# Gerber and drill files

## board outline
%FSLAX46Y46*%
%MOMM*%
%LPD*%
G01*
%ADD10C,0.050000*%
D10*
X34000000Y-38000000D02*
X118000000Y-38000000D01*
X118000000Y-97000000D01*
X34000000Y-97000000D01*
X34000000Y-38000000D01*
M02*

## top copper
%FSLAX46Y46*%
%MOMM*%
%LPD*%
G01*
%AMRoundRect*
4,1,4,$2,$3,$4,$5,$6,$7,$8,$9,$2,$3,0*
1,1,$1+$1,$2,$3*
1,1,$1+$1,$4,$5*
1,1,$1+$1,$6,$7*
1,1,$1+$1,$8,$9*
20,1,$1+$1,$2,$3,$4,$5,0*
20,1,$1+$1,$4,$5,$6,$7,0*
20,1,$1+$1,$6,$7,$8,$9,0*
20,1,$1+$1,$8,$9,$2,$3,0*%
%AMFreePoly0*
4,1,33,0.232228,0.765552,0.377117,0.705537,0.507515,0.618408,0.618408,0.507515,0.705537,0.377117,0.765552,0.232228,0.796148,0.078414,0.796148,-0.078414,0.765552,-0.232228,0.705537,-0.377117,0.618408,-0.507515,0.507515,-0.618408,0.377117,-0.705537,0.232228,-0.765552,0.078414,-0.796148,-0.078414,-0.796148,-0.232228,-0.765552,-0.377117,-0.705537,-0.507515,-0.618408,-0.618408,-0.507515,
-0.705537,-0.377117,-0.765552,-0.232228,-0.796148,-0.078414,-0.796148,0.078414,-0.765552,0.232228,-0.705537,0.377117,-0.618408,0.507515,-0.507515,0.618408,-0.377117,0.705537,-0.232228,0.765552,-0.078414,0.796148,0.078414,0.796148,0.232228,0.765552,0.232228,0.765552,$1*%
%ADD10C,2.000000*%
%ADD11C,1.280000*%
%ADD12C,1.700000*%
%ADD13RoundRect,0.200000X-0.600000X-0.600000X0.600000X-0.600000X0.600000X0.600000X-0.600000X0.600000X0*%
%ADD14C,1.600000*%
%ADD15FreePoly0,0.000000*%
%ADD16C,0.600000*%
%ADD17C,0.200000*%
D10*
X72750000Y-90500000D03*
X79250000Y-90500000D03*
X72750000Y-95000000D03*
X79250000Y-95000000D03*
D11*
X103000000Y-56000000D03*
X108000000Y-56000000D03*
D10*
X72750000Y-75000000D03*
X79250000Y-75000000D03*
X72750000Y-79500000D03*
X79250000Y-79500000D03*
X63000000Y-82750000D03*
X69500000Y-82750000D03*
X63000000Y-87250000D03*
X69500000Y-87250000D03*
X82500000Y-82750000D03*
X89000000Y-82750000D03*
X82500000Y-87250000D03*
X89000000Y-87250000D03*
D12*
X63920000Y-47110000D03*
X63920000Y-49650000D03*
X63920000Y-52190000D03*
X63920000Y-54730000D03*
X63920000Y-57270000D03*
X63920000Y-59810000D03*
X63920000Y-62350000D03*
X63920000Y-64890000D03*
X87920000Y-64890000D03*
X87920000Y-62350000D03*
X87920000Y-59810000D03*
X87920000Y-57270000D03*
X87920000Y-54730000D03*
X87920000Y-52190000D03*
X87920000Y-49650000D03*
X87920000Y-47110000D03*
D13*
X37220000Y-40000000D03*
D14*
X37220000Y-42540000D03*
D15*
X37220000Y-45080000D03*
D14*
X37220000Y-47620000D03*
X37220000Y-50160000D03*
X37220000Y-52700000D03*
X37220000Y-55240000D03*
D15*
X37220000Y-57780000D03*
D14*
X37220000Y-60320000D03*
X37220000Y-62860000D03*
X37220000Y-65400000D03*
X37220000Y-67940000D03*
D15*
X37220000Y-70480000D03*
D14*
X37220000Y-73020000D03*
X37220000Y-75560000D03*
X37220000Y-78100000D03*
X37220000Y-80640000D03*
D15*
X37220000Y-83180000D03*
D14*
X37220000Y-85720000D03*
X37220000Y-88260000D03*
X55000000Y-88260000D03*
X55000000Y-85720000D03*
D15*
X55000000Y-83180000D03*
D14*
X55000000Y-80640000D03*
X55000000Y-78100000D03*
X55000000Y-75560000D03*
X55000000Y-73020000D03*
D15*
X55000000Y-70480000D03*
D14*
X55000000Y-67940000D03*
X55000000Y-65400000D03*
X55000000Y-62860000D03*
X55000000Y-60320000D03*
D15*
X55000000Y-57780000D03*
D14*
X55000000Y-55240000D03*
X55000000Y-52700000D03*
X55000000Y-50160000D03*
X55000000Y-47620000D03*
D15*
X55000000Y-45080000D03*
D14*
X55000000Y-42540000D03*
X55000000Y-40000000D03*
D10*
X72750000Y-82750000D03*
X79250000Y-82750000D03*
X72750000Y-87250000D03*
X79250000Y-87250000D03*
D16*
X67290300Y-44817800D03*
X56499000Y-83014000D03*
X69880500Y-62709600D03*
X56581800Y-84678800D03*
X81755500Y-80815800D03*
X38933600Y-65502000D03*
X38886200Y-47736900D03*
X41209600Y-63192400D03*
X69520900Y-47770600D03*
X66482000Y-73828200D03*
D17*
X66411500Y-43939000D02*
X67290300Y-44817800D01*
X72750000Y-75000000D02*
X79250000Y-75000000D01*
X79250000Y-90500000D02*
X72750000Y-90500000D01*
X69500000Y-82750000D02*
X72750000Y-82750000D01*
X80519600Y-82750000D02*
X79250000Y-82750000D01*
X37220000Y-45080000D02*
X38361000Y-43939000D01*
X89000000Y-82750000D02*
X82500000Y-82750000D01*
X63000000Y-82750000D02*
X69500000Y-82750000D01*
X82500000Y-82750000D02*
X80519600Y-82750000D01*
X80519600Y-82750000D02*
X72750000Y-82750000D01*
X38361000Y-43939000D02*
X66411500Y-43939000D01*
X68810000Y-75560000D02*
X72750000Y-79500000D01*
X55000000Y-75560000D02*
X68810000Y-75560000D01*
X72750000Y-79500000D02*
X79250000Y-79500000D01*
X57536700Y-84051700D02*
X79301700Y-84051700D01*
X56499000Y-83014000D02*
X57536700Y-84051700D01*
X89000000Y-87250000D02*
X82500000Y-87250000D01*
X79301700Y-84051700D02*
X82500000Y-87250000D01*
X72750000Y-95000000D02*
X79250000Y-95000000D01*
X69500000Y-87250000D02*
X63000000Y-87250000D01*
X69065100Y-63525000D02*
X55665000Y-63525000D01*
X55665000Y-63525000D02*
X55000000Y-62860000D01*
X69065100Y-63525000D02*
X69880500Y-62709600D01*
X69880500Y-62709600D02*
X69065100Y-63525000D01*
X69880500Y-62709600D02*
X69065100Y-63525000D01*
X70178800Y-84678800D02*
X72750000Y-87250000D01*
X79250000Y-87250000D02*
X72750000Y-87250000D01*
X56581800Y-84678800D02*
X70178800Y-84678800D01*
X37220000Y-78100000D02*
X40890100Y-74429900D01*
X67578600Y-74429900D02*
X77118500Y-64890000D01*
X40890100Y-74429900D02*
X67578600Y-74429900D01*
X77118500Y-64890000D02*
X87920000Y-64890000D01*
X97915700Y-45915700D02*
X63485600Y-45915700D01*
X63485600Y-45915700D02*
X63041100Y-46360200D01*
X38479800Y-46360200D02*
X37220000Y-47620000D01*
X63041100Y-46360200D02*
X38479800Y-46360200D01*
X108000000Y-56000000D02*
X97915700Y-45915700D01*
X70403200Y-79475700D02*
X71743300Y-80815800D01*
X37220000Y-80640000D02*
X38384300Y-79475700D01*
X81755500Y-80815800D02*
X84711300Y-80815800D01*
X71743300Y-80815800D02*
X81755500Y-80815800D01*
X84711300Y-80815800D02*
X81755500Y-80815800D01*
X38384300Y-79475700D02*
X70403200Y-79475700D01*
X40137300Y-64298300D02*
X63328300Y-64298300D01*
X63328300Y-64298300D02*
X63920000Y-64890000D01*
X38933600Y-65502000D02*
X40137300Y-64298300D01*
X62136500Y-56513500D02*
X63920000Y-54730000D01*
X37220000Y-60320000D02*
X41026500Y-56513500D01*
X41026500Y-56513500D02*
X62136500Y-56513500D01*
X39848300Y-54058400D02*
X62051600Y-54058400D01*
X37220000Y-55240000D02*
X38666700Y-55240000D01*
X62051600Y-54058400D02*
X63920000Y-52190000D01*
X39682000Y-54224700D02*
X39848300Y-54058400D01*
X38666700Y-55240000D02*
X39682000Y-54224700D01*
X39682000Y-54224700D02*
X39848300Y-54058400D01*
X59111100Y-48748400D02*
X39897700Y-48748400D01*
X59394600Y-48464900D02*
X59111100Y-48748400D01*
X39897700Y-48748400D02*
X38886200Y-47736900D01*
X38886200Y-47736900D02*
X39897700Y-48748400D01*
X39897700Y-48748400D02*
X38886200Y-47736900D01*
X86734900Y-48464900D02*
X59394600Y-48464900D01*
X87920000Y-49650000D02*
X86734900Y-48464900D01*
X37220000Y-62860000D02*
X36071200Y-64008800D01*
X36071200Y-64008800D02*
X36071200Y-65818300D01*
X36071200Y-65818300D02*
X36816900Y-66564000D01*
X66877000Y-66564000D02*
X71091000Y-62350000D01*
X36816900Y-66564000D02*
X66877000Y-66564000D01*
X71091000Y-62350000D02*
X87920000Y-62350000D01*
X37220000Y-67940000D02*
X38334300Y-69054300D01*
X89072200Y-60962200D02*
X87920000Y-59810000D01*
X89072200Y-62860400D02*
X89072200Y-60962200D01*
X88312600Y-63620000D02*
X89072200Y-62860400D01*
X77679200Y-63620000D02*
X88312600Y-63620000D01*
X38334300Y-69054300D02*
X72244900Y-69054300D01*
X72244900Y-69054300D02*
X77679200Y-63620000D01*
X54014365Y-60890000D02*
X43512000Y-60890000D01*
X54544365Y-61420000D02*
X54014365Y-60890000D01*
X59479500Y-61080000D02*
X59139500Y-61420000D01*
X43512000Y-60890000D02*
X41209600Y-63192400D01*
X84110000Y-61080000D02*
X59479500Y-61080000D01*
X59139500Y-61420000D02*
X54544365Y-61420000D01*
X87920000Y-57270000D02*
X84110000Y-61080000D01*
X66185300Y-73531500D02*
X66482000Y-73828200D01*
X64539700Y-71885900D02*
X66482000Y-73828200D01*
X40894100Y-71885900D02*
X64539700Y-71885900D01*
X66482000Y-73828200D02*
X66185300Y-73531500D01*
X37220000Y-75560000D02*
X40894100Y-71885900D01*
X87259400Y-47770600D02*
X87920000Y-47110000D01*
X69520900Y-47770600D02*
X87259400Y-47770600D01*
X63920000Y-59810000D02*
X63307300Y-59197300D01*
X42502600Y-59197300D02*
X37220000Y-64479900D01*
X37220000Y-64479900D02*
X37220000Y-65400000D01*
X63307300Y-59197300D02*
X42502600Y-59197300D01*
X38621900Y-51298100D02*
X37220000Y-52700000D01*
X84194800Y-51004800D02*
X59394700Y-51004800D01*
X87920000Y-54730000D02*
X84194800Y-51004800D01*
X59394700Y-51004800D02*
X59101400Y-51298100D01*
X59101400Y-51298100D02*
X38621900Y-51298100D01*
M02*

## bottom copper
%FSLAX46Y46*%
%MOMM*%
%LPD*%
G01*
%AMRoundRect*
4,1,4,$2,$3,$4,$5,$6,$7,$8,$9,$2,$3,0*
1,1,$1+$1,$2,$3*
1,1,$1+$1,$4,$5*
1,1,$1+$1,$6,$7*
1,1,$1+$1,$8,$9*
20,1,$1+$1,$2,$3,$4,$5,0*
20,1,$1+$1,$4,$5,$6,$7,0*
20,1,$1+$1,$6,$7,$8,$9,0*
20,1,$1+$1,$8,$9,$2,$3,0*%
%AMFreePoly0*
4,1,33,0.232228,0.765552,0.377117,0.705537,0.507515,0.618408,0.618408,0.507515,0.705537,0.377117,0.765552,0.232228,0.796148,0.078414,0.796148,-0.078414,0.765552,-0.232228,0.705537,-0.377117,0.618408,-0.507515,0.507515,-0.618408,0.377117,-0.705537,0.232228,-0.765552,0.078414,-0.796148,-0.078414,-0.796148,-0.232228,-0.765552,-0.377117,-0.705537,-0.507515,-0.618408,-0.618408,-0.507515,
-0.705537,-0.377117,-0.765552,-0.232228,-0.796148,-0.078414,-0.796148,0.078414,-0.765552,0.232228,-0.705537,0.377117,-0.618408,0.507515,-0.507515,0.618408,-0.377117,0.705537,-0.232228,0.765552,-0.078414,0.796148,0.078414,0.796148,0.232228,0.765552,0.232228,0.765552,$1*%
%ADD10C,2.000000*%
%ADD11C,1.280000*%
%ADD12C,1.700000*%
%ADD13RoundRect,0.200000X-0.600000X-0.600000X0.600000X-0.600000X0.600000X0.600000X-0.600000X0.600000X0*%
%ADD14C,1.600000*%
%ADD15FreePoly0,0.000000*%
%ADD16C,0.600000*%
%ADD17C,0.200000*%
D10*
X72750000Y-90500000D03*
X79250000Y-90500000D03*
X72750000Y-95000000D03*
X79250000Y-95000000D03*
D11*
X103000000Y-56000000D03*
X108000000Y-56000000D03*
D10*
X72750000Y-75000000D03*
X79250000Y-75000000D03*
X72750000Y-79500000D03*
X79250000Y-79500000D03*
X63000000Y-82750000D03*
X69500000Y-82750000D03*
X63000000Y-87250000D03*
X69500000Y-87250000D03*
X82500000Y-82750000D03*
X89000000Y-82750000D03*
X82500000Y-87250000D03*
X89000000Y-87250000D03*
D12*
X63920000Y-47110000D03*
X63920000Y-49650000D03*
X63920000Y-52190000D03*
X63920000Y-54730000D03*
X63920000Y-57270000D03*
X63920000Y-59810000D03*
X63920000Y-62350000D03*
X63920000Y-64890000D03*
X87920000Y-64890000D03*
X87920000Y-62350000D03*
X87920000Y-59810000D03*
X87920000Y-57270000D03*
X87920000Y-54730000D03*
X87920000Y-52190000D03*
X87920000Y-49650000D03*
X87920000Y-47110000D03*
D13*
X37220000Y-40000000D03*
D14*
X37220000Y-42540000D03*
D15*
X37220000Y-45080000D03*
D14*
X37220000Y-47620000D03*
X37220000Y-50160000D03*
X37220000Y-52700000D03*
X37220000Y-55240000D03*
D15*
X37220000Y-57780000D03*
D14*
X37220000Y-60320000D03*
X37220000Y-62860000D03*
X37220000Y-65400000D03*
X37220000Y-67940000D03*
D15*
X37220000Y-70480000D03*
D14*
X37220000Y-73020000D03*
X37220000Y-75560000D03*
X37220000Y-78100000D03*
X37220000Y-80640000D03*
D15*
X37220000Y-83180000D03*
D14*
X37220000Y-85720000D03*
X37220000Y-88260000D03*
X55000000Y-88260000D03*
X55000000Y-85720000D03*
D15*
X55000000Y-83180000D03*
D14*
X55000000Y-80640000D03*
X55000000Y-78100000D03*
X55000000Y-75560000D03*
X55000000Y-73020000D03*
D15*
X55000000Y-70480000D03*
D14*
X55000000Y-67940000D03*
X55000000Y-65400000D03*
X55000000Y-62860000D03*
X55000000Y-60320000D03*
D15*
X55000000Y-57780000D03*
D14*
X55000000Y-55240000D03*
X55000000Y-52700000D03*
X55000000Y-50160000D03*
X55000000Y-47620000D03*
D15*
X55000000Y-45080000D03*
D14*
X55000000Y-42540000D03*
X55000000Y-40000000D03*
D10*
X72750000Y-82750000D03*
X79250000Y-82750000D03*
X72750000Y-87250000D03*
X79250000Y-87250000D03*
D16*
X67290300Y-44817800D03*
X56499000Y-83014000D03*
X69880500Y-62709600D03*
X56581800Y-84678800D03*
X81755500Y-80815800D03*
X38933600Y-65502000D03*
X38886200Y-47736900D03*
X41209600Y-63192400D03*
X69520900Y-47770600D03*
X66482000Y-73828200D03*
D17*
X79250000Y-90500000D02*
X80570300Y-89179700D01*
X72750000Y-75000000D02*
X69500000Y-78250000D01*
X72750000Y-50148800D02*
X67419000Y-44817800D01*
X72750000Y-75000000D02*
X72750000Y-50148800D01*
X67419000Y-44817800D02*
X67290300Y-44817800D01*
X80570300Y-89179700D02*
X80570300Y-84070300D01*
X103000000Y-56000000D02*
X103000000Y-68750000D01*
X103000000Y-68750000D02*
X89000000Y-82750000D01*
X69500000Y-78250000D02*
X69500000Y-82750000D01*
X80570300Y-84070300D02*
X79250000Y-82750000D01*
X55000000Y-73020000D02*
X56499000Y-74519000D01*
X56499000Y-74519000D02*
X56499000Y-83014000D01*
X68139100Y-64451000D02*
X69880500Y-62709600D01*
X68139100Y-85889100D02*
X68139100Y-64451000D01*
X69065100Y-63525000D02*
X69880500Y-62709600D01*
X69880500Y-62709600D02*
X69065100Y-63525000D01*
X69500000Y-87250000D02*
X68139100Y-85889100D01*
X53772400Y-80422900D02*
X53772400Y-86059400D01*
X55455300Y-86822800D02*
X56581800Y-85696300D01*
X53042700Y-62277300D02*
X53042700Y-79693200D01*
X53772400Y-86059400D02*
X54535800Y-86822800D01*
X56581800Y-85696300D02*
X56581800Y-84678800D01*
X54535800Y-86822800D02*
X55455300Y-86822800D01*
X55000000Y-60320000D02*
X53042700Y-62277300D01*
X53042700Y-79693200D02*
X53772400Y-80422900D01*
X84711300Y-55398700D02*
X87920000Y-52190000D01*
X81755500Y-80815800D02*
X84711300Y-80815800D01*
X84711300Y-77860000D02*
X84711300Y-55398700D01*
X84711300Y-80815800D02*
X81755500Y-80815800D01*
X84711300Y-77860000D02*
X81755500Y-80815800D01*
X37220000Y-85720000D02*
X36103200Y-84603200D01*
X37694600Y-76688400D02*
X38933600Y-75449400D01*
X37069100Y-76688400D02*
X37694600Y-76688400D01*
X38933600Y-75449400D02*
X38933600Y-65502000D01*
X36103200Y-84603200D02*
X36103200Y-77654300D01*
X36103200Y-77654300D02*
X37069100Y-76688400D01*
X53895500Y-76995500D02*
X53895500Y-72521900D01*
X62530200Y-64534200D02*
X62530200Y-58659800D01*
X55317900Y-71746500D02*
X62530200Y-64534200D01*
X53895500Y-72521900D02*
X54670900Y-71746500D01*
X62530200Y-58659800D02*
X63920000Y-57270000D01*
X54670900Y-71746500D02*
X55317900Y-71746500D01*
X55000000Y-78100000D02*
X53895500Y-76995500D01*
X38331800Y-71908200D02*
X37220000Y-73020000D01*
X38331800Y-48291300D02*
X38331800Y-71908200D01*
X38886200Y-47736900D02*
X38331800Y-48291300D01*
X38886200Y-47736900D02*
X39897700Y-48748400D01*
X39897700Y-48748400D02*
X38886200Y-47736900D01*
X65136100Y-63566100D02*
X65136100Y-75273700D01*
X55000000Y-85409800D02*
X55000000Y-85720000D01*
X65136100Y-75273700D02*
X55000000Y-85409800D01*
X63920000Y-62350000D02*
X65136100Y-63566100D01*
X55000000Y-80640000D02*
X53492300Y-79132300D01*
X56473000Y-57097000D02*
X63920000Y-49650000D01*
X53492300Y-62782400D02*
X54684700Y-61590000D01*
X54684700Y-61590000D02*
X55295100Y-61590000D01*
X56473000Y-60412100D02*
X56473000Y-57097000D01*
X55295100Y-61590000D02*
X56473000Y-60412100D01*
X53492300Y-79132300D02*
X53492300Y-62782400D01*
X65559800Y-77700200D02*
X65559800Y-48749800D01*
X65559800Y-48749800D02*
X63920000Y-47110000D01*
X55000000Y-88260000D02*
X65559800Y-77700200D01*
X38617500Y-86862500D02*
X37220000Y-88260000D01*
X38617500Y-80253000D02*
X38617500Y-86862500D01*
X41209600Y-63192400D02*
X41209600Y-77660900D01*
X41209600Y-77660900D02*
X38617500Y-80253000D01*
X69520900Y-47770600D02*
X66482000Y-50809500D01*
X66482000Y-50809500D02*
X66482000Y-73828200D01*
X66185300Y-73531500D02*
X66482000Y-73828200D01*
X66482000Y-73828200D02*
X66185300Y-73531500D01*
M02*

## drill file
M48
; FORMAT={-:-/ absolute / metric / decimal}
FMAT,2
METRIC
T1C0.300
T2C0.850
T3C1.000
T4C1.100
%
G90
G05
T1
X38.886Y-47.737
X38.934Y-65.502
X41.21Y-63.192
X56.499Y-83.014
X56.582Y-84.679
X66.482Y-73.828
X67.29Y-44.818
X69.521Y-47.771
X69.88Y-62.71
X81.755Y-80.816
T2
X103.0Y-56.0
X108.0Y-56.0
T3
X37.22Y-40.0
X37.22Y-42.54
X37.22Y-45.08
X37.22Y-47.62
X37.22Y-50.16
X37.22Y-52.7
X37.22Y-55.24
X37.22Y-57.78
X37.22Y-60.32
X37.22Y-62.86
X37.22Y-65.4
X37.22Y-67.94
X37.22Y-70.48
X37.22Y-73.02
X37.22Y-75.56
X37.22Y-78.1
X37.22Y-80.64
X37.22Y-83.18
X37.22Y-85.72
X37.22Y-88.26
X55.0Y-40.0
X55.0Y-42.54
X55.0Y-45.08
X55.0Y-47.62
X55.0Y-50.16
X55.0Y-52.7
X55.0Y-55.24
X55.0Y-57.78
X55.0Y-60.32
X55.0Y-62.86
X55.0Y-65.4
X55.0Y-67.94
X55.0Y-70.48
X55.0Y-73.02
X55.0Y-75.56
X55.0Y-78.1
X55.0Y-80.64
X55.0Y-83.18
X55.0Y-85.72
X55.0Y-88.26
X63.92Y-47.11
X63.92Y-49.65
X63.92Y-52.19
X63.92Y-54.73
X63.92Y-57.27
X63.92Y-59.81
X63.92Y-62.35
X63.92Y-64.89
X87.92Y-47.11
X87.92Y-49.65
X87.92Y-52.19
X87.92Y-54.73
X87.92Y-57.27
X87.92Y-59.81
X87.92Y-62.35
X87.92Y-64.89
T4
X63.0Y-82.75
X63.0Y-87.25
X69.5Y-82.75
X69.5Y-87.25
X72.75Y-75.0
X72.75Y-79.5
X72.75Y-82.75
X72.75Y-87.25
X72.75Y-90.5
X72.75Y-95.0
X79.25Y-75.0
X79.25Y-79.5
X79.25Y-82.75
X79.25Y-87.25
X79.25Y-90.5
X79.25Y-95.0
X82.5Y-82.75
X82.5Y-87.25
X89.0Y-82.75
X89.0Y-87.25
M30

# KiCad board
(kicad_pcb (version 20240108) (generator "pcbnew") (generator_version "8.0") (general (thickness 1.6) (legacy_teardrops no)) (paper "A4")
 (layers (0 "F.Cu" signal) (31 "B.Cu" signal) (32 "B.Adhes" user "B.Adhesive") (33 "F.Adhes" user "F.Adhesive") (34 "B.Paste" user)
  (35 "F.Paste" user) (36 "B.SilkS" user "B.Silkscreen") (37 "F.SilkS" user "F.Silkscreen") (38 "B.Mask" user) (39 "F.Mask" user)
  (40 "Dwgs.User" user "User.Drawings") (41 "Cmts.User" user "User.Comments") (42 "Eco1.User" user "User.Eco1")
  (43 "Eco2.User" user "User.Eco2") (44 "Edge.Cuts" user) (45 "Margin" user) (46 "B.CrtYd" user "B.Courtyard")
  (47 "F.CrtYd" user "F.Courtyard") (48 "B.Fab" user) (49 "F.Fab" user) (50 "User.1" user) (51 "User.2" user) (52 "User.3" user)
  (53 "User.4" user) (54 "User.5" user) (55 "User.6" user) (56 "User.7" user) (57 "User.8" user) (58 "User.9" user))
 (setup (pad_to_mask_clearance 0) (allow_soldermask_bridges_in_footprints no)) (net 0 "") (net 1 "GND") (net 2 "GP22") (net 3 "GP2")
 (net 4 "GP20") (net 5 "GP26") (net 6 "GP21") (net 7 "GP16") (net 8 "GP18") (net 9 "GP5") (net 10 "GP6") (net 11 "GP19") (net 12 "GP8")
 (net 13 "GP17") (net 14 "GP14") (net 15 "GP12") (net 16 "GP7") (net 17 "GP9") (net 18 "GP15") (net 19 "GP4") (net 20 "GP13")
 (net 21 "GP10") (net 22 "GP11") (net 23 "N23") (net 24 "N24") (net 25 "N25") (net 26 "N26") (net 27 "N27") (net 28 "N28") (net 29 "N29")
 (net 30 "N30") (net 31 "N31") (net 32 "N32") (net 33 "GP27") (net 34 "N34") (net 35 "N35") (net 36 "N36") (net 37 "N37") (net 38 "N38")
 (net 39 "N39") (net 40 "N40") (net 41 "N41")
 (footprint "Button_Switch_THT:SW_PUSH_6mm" (layer "F.Cu") (at 72.75 90.5)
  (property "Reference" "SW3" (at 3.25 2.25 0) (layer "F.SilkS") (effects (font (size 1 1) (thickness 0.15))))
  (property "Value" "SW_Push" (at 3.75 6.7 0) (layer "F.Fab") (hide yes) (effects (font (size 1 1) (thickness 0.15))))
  (pad "1" thru_hole circle (at 0 0 90) (size 2 2) (drill 1.1) (layers "*.Cu" "*.Mask") (remove_unused_layers no) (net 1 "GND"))
  (pad "1" thru_hole circle (at 6.5 0 90) (size 2 2) (drill 1.1) (layers "*.Cu" "*.Mask") (remove_unused_layers no) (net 1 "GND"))
  (pad "2" thru_hole circle (at 0 4.5 90) (size 2 2) (drill 1.1) (layers "*.Cu" "*.Mask") (remove_unused_layers no) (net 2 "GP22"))
  (pad "2" thru_hole circle (at 6.5 4.5 90) (size 2 2) (drill 1.1) (layers "*.Cu" "*.Mask") (remove_unused_layers no) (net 2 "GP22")))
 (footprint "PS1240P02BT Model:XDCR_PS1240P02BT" (layer "F.Cu") (at 105.5 56)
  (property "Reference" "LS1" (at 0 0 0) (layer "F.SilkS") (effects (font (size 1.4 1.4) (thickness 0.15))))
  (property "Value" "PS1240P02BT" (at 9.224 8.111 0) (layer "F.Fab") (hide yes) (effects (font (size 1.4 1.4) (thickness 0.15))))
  (pad "1" thru_hole circle (at -2.5 0) (size 1.28 1.28) (drill 0.85) (layers "*.Cu" "*.Mask") (remove_unused_layers no) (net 1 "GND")
   (solder_mask_margin 0.102))
  (pad "2" thru_hole circle (at 2.5 0) (size 1.28 1.28) (drill 0.85) (layers "*.Cu" "*.Mask") (remove_unused_layers no) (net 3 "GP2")
   (solder_mask_margin 0.102)))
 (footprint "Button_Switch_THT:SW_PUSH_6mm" (layer "F.Cu") (at 72.75 75)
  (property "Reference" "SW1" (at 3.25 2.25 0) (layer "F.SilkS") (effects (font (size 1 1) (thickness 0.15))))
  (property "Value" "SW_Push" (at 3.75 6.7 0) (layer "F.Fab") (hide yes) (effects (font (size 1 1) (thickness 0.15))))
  (pad "1" thru_hole circle (at 0 0 90) (size 2 2) (drill 1.1) (layers "*.Cu" "*.Mask") (remove_unused_layers no) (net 1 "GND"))
  (pad "1" thru_hole circle (at 6.5 0 90) (size 2 2) (drill 1.1) (layers "*.Cu" "*.Mask") (remove_unused_layers no) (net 1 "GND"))
  (pad "2" thru_hole circle (at 0 4.5 90) (size 2 2) (drill 1.1) (layers "*.Cu" "*.Mask") (remove_unused_layers no) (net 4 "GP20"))
  (pad "2" thru_hole circle (at 6.5 4.5 90) (size 2 2) (drill 1.1) (layers "*.Cu" "*.Mask") (remove_unused_layers no) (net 4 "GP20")))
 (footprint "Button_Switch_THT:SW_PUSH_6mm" (layer "F.Cu") (at 63 82.75)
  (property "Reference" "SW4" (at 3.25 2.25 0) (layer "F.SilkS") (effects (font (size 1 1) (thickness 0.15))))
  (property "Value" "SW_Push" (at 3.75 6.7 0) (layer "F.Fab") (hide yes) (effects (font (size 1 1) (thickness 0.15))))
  (pad "1" thru_hole circle (at 0 0 90) (size 2 2) (drill 1.1) (layers "*.Cu" "*.Mask") (remove_unused_layers no) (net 1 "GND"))
  (pad "1" thru_hole circle (at 6.5 0 90) (size 2 2) (drill 1.1) (layers "*.Cu" "*.Mask") (remove_unused_layers no) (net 1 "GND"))
  (pad "2" thru_hole circle (at 0 4.5 90) (size 2 2) (drill 1.1) (layers "*.Cu" "*.Mask") (remove_unused_layers no) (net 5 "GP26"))
  (pad "2" thru_hole circle (at 6.5 4.5 90) (size 2 2) (drill 1.1) (layers "*.Cu" "*.Mask") (remove_unused_layers no) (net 5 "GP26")))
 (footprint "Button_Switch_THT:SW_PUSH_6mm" (layer "F.Cu") (at 82.5 82.75)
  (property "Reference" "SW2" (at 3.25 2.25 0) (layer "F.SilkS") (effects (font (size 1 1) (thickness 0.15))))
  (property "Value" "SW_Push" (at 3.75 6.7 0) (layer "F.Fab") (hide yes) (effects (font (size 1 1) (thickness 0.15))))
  (pad "1" thru_hole circle (at 0 0 90) (size 2 2) (drill 1.1) (layers "*.Cu" "*.Mask") (remove_unused_layers no) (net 1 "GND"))
  (pad "1" thru_hole circle (at 6.5 0 90) (size 2 2) (drill 1.1) (layers "*.Cu" "*.Mask") (remove_unused_layers no) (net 1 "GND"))
  (pad "2" thru_hole circle (at 0 4.5 90) (size 2 2) (drill 1.1) (layers "*.Cu" "*.Mask") (remove_unused_layers no) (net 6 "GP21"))
  (pad "2" thru_hole circle (at 6.5 4.5 90) (size 2 2) (drill 1.1) (layers "*.Cu" "*.Mask") (remove_unused_layers no) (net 6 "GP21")))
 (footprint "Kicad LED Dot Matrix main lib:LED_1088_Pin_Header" (layer "F.Cu") (at 60 40)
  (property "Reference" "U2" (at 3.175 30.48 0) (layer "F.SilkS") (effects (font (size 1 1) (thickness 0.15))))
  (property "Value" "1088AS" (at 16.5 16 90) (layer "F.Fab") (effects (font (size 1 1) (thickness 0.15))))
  (pad "1" thru_hole circle (at 3.92 7.11 270) (size 1.7 1.7) (drill 1) (layers "*.Cu" "*.Mask") (remove_unused_layers no) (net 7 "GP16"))
  (pad "2" thru_hole circle (at 3.92 9.65 270) (size 1.7 1.7) (drill 1) (layers "*.Cu" "*.Mask") (remove_unused_layers no) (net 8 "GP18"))
  (pad "3" thru_hole circle (at 3.92 12.19 270) (size 1.7 1.7) (drill 1) (layers "*.Cu" "*.Mask") (remove_unused_layers no) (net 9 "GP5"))
  (pad "4" thru_hole circle (at 3.92 14.73 270) (size 1.7 1.7) (drill 1) (layers "*.Cu" "*.Mask") (remove_unused_layers no) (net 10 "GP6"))
  (pad "5" thru_hole circle (at 3.92 17.27 270) (size 1.7 1.7) (drill 1) (layers "*.Cu" "*.Mask") (remove_unused_layers no) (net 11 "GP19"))
  (pad "6" thru_hole circle (at 3.92 19.81 270) (size 1.7 1.7) (drill 1) (layers "*.Cu" "*.Mask") (remove_unused_layers no) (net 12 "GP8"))
  (pad "7" thru_hole circle (at 3.92 22.35 270) (size 1.7 1.7) (drill 1) (layers "*.Cu" "*.Mask") (remove_unused_layers no) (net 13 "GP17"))
  (pad "8" thru_hole circle (at 3.92 24.89 270) (size 1.7 1.7) (drill 1) (layers "*.Cu" "*.Mask") (remove_unused_layers no) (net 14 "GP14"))
  (pad "9" thru_hole circle (at 27.92 24.89 270) (size 1.7 1.7) (drill 1) (layers "*.Cu" "*.Mask") (remove_unused_layers no) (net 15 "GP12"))
  (pad "10" thru_hole circle (at 27.92 22.35 270) (size 1.7 1.7) (drill 1) (layers "*.Cu" "*.Mask") (remove_unused_layers no) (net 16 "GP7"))
  (pad "11" thru_hole circle (at 27.92 19.81 270) (size 1.7 1.7) (drill 1) (layers "*.Cu" "*.Mask") (remove_unused_layers no) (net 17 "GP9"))
  (pad "12" thru_hole circle (at 27.92 17.27 270) (size 1.7 1.7) (drill 1) (layers "*.Cu" "*.Mask") (remove_unused_layers no)
   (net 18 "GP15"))
  (pad "13" thru_hole circle (at 27.92 14.73 270) (size 1.7 1.7) (drill 1) (layers "*.Cu" "*.Mask") (remove_unused_layers no) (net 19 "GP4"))
  (pad "14" thru_hole circle (at 27.92 12.19 270) (size 1.7 1.7) (drill 1) (layers "*.Cu" "*.Mask") (remove_unused_layers no)
   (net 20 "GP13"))
  (pad "15" thru_hole circle (at 27.92 9.65 270) (size 1.7 1.7) (drill 1) (layers "*.Cu" "*.Mask") (remove_unused_layers no) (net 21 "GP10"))
  (pad "16" thru_hole circle (at 27.92 7.11 270) (size 1.7 1.7) (drill 1) (layers "*.Cu" "*.Mask") (remove_unused_layers no) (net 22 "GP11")))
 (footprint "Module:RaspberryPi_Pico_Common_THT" (layer "F.Cu") (at 37.22 40)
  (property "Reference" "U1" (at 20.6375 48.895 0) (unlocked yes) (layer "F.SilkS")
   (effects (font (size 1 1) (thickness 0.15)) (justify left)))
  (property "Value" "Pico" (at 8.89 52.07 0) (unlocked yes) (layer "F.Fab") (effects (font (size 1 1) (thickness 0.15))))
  (pad "1" thru_hole roundrect (at 0 0) (size 1.6 1.6) (drill 1) (layers "*.Cu" "*.Mask") (remove_unused_layers no) (roundrect_rratio 0.125)
   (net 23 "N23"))
  (pad "2" thru_hole circle (at 0 2.54) (size 1.6 1.6) (drill 1) (layers "*.Cu" "*.Mask") (remove_unused_layers no) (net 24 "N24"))
  (pad "3" thru_hole custom (at 0 5.08) (size 1.6 1.6) (drill 1) (layers "*.Cu" "*.Mask") (remove_unused_layers no) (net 1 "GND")
   (options (clearance outline) (anchor circle)) (primitives))
  (pad "4" thru_hole circle (at 0 7.62) (size 1.6 1.6) (drill 1) (layers "*.Cu" "*.Mask") (remove_unused_layers no) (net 3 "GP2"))
  (pad "5" thru_hole circle (at 0 10.16) (size 1.6 1.6) (drill 1) (layers "*.Cu" "*.Mask") (remove_unused_layers no) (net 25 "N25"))
  (pad "6" thru_hole circle (at 0 12.7) (size 1.6 1.6) (drill 1) (layers "*.Cu" "*.Mask") (remove_unused_layers no) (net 19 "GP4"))
  (pad "7" thru_hole circle (at 0 15.24) (size 1.6 1.6) (drill 1) (layers "*.Cu" "*.Mask") (remove_unused_layers no) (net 9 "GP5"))
  (pad "8" thru_hole custom (at 0 17.78) (size 1.6 1.6) (drill 1) (layers "*.Cu" "*.Mask") (remove_unused_layers no) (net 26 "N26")
   (options (clearance outline) (anchor circle)) (primitives))
  (pad "9" thru_hole circle (at 0 20.32) (size 1.6 1.6) (drill 1) (layers "*.Cu" "*.Mask") (remove_unused_layers no) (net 10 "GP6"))
  (pad "10" thru_hole circle (at 0 22.86) (size 1.6 1.6) (drill 1) (layers "*.Cu" "*.Mask") (remove_unused_layers no) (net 16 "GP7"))
  (pad "11" thru_hole circle (at 0 25.4) (size 1.6 1.6) (drill 1) (layers "*.Cu" "*.Mask") (remove_unused_layers no) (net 12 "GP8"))
  (pad "12" thru_hole circle (at 0 27.94) (size 1.6 1.6) (drill 1) (layers "*.Cu" "*.Mask") (remove_unused_layers no) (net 17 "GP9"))
  (pad "13" thru_hole custom (at 0 30.48) (size 1.6 1.6) (drill 1) (layers "*.Cu" "*.Mask") (remove_unused_layers no) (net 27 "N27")
   (options (clearance outline) (anchor circle)) (primitives))
  (pad "14" thru_hole circle (at 0 33.02) (size 1.6 1.6) (drill 1) (layers "*.Cu" "*.Mask") (remove_unused_layers no) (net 21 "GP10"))
  (pad "15" thru_hole circle (at 0 35.56) (size 1.6 1.6) (drill 1) (layers "*.Cu" "*.Mask") (remove_unused_layers no) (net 22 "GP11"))
  (pad "16" thru_hole circle (at 0 38.1) (size 1.6 1.6) (drill 1) (layers "*.Cu" "*.Mask") (remove_unused_layers no) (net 15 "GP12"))
  (pad "17" thru_hole circle (at 0 40.64) (size 1.6 1.6) (drill 1) (layers "*.Cu" "*.Mask") (remove_unused_layers no) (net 20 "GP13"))
  (pad "18" thru_hole custom (at 0 43.18) (size 1.6 1.6) (drill 1) (layers "*.Cu" "*.Mask") (remove_unused_layers no) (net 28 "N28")
   (options (clearance outline) (anchor circle)) (primitives))
  (pad "19" thru_hole circle (at 0 45.72) (size 1.6 1.6) (drill 1) (layers "*.Cu" "*.Mask") (remove_unused_layers no) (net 14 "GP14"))
  (pad "20" thru_hole circle (at 0 48.26) (size 1.6 1.6) (drill 1) (layers "*.Cu" "*.Mask") (remove_unused_layers no) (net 18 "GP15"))
  (pad "21" thru_hole circle (at 17.78 48.26) (size 1.6 1.6) (drill 1) (layers "*.Cu" "*.Mask") (remove_unused_layers no) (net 7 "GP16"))
  (pad "22" thru_hole circle (at 17.78 45.72) (size 1.6 1.6) (drill 1) (layers "*.Cu" "*.Mask") (remove_unused_layers no) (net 13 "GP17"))
  (pad "23" thru_hole custom (at 17.78 43.18) (size 1.6 1.6) (drill 1) (layers "*.Cu" "*.Mask") (remove_unused_layers no) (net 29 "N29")
   (options (clearance outline) (anchor circle)) (primitives))
  (pad "24" thru_hole circle (at 17.78 40.64) (size 1.6 1.6) (drill 1) (layers "*.Cu" "*.Mask") (remove_unused_layers no) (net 8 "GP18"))
  (pad "25" thru_hole circle (at 17.78 38.1) (size 1.6 1.6) (drill 1) (layers "*.Cu" "*.Mask") (remove_unused_layers no) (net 11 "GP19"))
  (pad "26" thru_hole circle (at 17.78 35.56) (size 1.6 1.6) (drill 1) (layers "*.Cu" "*.Mask") (remove_unused_layers no) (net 4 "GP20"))
  (pad "27" thru_hole circle (at 17.78 33.02) (size 1.6 1.6) (drill 1) (layers "*.Cu" "*.Mask") (remove_unused_layers no) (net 6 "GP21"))
  (pad "28" thru_hole custom (at 17.78 30.48) (size 1.6 1.6) (drill 1) (layers "*.Cu" "*.Mask") (remove_unused_layers no) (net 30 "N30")
   (options (clearance outline) (anchor circle)) (primitives))
  (pad "29" thru_hole circle (at 17.78 27.94) (size 1.6 1.6) (drill 1) (layers "*.Cu" "*.Mask") (remove_unused_layers no) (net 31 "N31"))
  (pad "30" thru_hole circle (at 17.78 25.4) (size 1.6 1.6) (drill 1) (layers "*.Cu" "*.Mask") (remove_unused_layers no) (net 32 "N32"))
  (pad "31" thru_hole circle (at 17.78 22.86) (size 1.6 1.6) (drill 1) (layers "*.Cu" "*.Mask") (remove_unused_layers no) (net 5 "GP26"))
  (pad "32" thru_hole circle (at 17.78 20.32) (size 1.6 1.6) (drill 1) (layers "*.Cu" "*.Mask") (remove_unused_layers no) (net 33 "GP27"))
  (pad "33" thru_hole custom (at 17.78 17.78) (size 1.6 1.6) (drill 1) (layers "*.Cu" "*.Mask") (remove_unused_layers no) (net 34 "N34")
   (options (clearance outline) (anchor circle)) (primitives))
  (pad "34" thru_hole circle (at 17.78 15.24) (size 1.6 1.6) (drill 1) (layers "*.Cu" "*.Mask") (remove_unused_layers no) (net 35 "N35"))
  (pad "35" thru_hole circle (at 17.78 12.7) (size 1.6 1.6) (drill 1) (layers "*.Cu" "*.Mask") (remove_unused_layers no) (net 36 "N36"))
  (pad "36" thru_hole circle (at 17.78 10.16) (size 1.6 1.6) (drill 1) (layers "*.Cu" "*.Mask") (remove_unused_layers no) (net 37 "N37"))
  (pad "37" thru_hole circle (at 17.78 7.62) (size 1.6 1.6) (drill 1) (layers "*.Cu" "*.Mask") (remove_unused_layers no) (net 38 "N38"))
  (pad "38" thru_hole custom (at 17.78 5.08) (size 1.6 1.6) (drill 1) (layers "*.Cu" "*.Mask") (remove_unused_layers no) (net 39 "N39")
   (options (clearance outline) (anchor circle)) (primitives))
  (pad "39" thru_hole circle (at 17.78 2.54) (size 1.6 1.6) (drill 1) (layers "*.Cu" "*.Mask") (remove_unused_layers no) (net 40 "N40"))
  (pad "40" thru_hole circle (at 17.78 0) (size 1.6 1.6) (drill 1) (layers "*.Cu" "*.Mask") (remove_unused_layers no) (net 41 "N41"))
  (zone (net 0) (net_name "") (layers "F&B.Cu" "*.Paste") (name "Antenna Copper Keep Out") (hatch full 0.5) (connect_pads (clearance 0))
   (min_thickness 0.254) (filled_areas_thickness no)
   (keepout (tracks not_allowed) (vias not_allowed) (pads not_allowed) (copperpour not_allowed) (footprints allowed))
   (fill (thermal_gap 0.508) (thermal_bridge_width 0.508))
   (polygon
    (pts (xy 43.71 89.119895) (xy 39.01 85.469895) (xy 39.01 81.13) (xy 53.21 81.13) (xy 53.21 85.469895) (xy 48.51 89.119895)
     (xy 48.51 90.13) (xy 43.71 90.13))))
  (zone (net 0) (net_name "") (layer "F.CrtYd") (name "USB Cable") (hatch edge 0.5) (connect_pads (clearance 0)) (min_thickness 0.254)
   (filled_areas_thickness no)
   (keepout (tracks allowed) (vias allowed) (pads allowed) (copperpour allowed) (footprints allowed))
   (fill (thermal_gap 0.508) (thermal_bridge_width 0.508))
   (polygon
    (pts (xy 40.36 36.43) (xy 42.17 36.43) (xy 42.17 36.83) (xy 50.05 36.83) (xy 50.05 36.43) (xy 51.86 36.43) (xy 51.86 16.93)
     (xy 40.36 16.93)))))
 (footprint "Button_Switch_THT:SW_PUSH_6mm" (layer "F.Cu") (at 72.75 82.75)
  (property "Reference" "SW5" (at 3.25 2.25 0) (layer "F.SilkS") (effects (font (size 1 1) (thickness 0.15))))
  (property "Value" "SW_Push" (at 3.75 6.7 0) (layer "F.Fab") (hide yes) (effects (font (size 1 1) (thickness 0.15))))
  (pad "1" thru_hole circle (at 0 0 90) (size 2 2) (drill 1.1) (layers "*.Cu" "*.Mask") (remove_unused_layers no) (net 1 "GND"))
  (pad "1" thru_hole circle (at 6.5 0 90) (size 2 2) (drill 1.1) (layers "*.Cu" "*.Mask") (remove_unused_layers no) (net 1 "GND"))
  (pad "2" thru_hole circle (at 0 4.5 90) (size 2 2) (drill 1.1) (layers "*.Cu" "*.Mask") (remove_unused_layers no) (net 33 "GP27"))
  (pad "2" thru_hole circle (at 6.5 4.5 90) (size 2 2) (drill 1.1) (layers "*.Cu" "*.Mask") (remove_unused_layers no) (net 33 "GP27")))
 (gr_rect (start 34 38) (end 118 97) (stroke (width 0.05) (type default)) (fill none) (layer "Edge.Cuts"))
 (segment (start 66.4115 43.939) (end 67.2903 44.8178) (width 0.2) (layer "F.Cu") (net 1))
 (segment (start 72.75 75) (end 79.25 75) (width 0.2) (layer "F.Cu") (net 1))
 (segment (start 79.25 90.5) (end 72.75 90.5) (width 0.2) (layer "F.Cu") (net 1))
 (segment (start 69.5 82.75) (end 72.75 82.75) (width 0.2) (layer "F.Cu") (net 1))
 (segment (start 80.5196 82.75) (end 79.25 82.75) (width 0.2) (layer "F.Cu") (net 1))
 (segment (start 37.22 45.08) (end 38.361 43.939) (width 0.2) (layer "F.Cu") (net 1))
 (segment (start 89 82.75) (end 82.5 82.75) (width 0.2) (layer "F.Cu") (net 1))
 (segment (start 63 82.75) (end 69.5 82.75) (width 0.2) (layer "F.Cu") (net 1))
 (segment (start 82.5 82.75) (end 80.5196 82.75) (width 0.2) (layer "F.Cu") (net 1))
 (segment (start 80.5196 82.75) (end 72.75 82.75) (width 0.2) (layer "F.Cu") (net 1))
 (segment (start 38.361 43.939) (end 66.4115 43.939) (width 0.2) (layer "F.Cu") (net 1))
 (via (at 67.2903 44.8178) (size 0.6) (drill 0.3) (layers "F.Cu" "B.Cu") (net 1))
 (segment (start 79.25 90.5) (end 80.5703 89.1797) (width 0.2) (layer "B.Cu") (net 1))
 (segment (start 72.75 75) (end 69.5 78.25) (width 0.2) (layer "B.Cu") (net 1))
 (segment (start 72.75 50.1488) (end 67.419 44.8178) (width 0.2) (layer "B.Cu") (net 1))
 (segment (start 72.75 75) (end 72.75 50.1488) (width 0.2) (layer "B.Cu") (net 1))
 (segment (start 67.419 44.8178) (end 67.2903 44.8178) (width 0.2) (layer "B.Cu") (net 1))
 (segment (start 80.5703 89.1797) (end 80.5703 84.0703) (width 0.2) (layer "B.Cu") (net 1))
 (segment (start 103 56) (end 103 68.75) (width 0.2) (layer "B.Cu") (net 1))
 (segment (start 103 68.75) (end 89 82.75) (width 0.2) (layer "B.Cu") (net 1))
 (segment (start 69.5 78.25) (end 69.5 82.75) (width 0.2) (layer "B.Cu") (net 1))
 (segment (start 80.5703 84.0703) (end 79.25 82.75) (width 0.2) (layer "B.Cu") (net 1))
 (segment (start 68.81 75.56) (end 72.75 79.5) (width 0.2) (layer "F.Cu") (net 4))
 (segment (start 55 75.56) (end 68.81 75.56) (width 0.2) (layer "F.Cu") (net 4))
 (segment (start 72.75 79.5) (end 79.25 79.5) (width 0.2) (layer "F.Cu") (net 4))
 (segment (start 57.5367 84.0517) (end 79.3017 84.0517) (width 0.2) (layer "F.Cu") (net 6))
 (segment (start 56.499 83.014) (end 57.5367 84.0517) (width 0.2) (layer "F.Cu") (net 6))
 (segment (start 89 87.25) (end 82.5 87.25) (width 0.2) (layer "F.Cu") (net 6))
 (segment (start 79.3017 84.0517) (end 82.5 87.25) (width 0.2) (layer "F.Cu") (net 6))
 (via (at 56.499 83.014) (size 0.6) (drill 0.3) (layers "F.Cu" "B.Cu") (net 6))
 (segment (start 55 73.02) (end 56.499 74.519) (width 0.2) (layer "B.Cu") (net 6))
 (segment (start 56.499 74.519) (end 56.499 83.014) (width 0.2) (layer "B.Cu") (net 6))
 (segment (start 72.75 95) (end 79.25 95) (width 0.2) (layer "F.Cu") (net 2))
 (segment (start 69.5 87.25) (end 63 87.25) (width 0.2) (layer "F.Cu") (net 5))
 (segment (start 69.0651 63.525) (end 55.665 63.525) (width 0.2) (layer "F.Cu") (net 5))
 (segment (start 55.665 63.525) (end 55 62.86) (width 0.2) (layer "F.Cu") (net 5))
 (segment (start 69.0651 63.525) (end 69.8805 62.7096) (width 0.2) (layer "F.Cu") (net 5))
 (segment (start 69.8805 62.7096) (end 69.0651 63.525) (width 0.2) (layer "F.Cu") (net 5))
 (segment (start 69.8805 62.7096) (end 69.0651 63.525) (width 0.2) (layer "F.Cu") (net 5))
 (via (at 69.8805 62.7096) (size 0.6) (drill 0.3) (layers "F.Cu" "B.Cu") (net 5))
 (segment (start 68.1391 64.451) (end 69.8805 62.7096) (width 0.2) (layer "B.Cu") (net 5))
 (segment (start 68.1391 85.8891) (end 68.1391 64.451) (width 0.2) (layer "B.Cu") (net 5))
 (segment (start 69.0651 63.525) (end 69.8805 62.7096) (width 0.2) (layer "B.Cu") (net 5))
 (segment (start 69.8805 62.7096) (end 69.0651 63.525) (width 0.2) (layer "B.Cu") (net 5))
 (segment (start 69.5 87.25) (end 68.1391 85.8891) (width 0.2) (layer "B.Cu") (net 5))
 (segment (start 70.1788 84.6788) (end 72.75 87.25) (width 0.2) (layer "F.Cu") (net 33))
 (segment (start 79.25 87.25) (end 72.75 87.25) (width 0.2) (layer "F.Cu") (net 33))
 (segment (start 56.5818 84.6788) (end 70.1788 84.6788) (width 0.2) (layer "F.Cu") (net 33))
 (via (at 56.5818 84.6788) (size 0.6) (drill 0.3) (layers "F.Cu" "B.Cu") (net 33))
 (segment (start 53.7724 80.4229) (end 53.7724 86.0594) (width 0.2) (layer "B.Cu") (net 33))
 (segment (start 55.4553 86.8228) (end 56.5818 85.6963) (width 0.2) (layer "B.Cu") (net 33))
 (segment (start 53.0427 62.2773) (end 53.0427 79.6932) (width 0.2) (layer "B.Cu") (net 33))
 (segment (start 53.7724 86.0594) (end 54.5358 86.8228) (width 0.2) (layer "B.Cu") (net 33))
 (segment (start 56.5818 85.6963) (end 56.5818 84.6788) (width 0.2) (layer "B.Cu") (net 33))
 (segment (start 54.5358 86.8228) (end 55.4553 86.8228) (width 0.2) (layer "B.Cu") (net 33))
 (segment (start 55 60.32) (end 53.0427 62.2773) (width 0.2) (layer "B.Cu") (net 33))
 (segment (start 53.0427 79.6932) (end 53.7724 80.4229) (width 0.2) (layer "B.Cu") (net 33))
 (segment (start 37.22 78.1) (end 40.8901 74.4299) (width 0.2) (layer "F.Cu") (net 15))
 (segment (start 67.5786 74.4299) (end 77.1185 64.89) (width 0.2) (layer "F.Cu") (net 15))
 (segment (start 40.8901 74.4299) (end 67.5786 74.4299) (width 0.2) (layer "F.Cu") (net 15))
 (segment (start 77.1185 64.89) (end 87.92 64.89) (width 0.2) (layer "F.Cu") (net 15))
 (segment (start 97.9157 45.9157) (end 63.4856 45.9157) (width 0.2) (layer "F.Cu") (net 3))
 (segment (start 63.4856 45.9157) (end 63.0411 46.3602) (width 0.2) (layer "F.Cu") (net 3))
 (segment (start 38.4798 46.3602) (end 37.22 47.62) (width 0.2) (layer "F.Cu") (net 3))
 (segment (start 63.0411 46.3602) (end 38.4798 46.3602) (width 0.2) (layer "F.Cu") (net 3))
 (segment (start 108 56) (end 97.9157 45.9157) (width 0.2) (layer "F.Cu") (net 3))
 (segment (start 70.4032 79.4757) (end 71.7433 80.8158) (width 0.2) (layer "F.Cu") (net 20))
 (segment (start 37.22 80.64) (end 38.3843 79.4757) (width 0.2) (layer "F.Cu") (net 20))
 (segment (start 81.7555 80.8158) (end 84.7113 80.8158) (width 0.2) (layer "F.Cu") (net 20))
 (segment (start 71.7433 80.8158) (end 81.7555 80.8158) (width 0.2) (layer "F.Cu") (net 20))
 (segment (start 84.7113 80.8158) (end 81.7555 80.8158) (width 0.2) (layer "F.Cu") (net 20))
 (segment (start 38.3843 79.4757) (end 70.4032 79.4757) (width 0.2) (layer "F.Cu") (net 20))
 (via (at 81.7555 80.8158) (size 0.6) (drill 0.3) (layers "F.Cu" "B.Cu") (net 20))
 (segment (start 84.7113 55.3987) (end 87.92 52.19) (width 0.2) (layer "B.Cu") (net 20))
 (segment (start 81.7555 80.8158) (end 84.7113 80.8158) (width 0.2) (layer "B.Cu") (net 20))
 (segment (start 84.7113 77.86) (end 84.7113 55.3987) (width 0.2) (layer "B.Cu") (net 20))
 (segment (start 84.7113 80.8158) (end 81.7555 80.8158) (width 0.2) (layer "B.Cu") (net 20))
 (segment (start 84.7113 77.86) (end 81.7555 80.8158) (width 0.2) (layer "B.Cu") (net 20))
 (segment (start 40.1373 64.2983) (end 63.3283 64.2983) (width 0.2) (layer "F.Cu") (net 14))
 (segment (start 63.3283 64.2983) (end 63.92 64.89) (width 0.2) (layer "F.Cu") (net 14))
 (segment (start 38.9336 65.502) (end 40.1373 64.2983) (width 0.2) (layer "F.Cu") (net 14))
 (via (at 38.9336 65.502) (size 0.6) (drill 0.3) (layers "F.Cu" "B.Cu") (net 14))
 (segment (start 37.22 85.72) (end 36.1032 84.6032) (width 0.2) (layer "B.Cu") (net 14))
 (segment (start 37.6946 76.6884) (end 38.9336 75.4494) (width 0.2) (layer "B.Cu") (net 14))
 (segment (start 37.0691 76.6884) (end 37.6946 76.6884) (width 0.2) (layer "B.Cu") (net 14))
 (segment (start 38.9336 75.4494) (end 38.9336 65.502) (width 0.2) (layer "B.Cu") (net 14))
 (segment (start 36.1032 84.6032) (end 36.1032 77.6543) (width 0.2) (layer "B.Cu") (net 14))
 (segment (start 36.1032 77.6543) (end 37.0691 76.6884) (width 0.2) (layer "B.Cu") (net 14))
 (segment (start 62.1365 56.5135) (end 63.92 54.73) (width 0.2) (layer "F.Cu") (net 10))
 (segment (start 37.22 60.32) (end 41.0265 56.5135) (width 0.2) (layer "F.Cu") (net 10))
 (segment (start 41.0265 56.5135) (end 62.1365 56.5135) (width 0.2) (layer "F.Cu") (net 10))
 (segment (start 39.8483 54.0584) (end 62.0516 54.0584) (width 0.2) (layer "F.Cu") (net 9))
 (segment (start 37.22 55.24) (end 38.6667 55.24) (width 0.2) (layer "F.Cu") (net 9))
 (segment (start 62.0516 54.0584) (end 63.92 52.19) (width 0.2) (layer "F.Cu") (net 9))
 (segment (start 39.682 54.2247) (end 39.8483 54.0584) (width 0.2) (layer "F.Cu") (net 9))
 (segment (start 38.6667 55.24) (end 39.682 54.2247) (width 0.2) (layer "F.Cu") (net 9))
 (segment (start 39.682 54.2247) (end 39.8483 54.0584) (width 0.2) (layer "F.Cu") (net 9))
 (segment (start 53.8955 76.9955) (end 53.8955 72.5219) (width 0.2) (layer "B.Cu") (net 11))
 (segment (start 62.5302 64.5342) (end 62.5302 58.6598) (width 0.2) (layer "B.Cu") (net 11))
 (segment (start 55.3179 71.7465) (end 62.5302 64.5342) (width 0.2) (layer "B.Cu") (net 11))
 (segment (start 53.8955 72.5219) (end 54.6709 71.7465) (width 0.2) (layer "B.Cu") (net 11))
 (segment (start 62.5302 58.6598) (end 63.92 57.27) (width 0.2) (layer "B.Cu") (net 11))
 (segment (start 54.6709 71.7465) (end 55.3179 71.7465) (width 0.2) (layer "B.Cu") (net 11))
 (segment (start 55 78.1) (end 53.8955 76.9955) (width 0.2) (layer "B.Cu") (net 11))
 (segment (start 59.1111 48.7484) (end 39.8977 48.7484) (width 0.2) (layer "F.Cu") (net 21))
 (segment (start 59.3946 48.4649) (end 59.1111 48.7484) (width 0.2) (layer "F.Cu") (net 21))
 (segment (start 39.8977 48.7484) (end 38.8862 47.7369) (width 0.2) (layer "F.Cu") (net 21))
 (segment (start 38.8862 47.7369) (end 39.8977 48.7484) (width 0.2) (layer "F.Cu") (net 21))
 (segment (start 39.8977 48.7484) (end 38.8862 47.7369) (width 0.2) (layer "F.Cu") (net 21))
 (segment (start 86.7349 48.4649) (end 59.3946 48.4649) (width 0.2) (layer "F.Cu") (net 21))
 (segment (start 87.92 49.65) (end 86.7349 48.4649) (width 0.2) (layer "F.Cu") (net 21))
 (via (at 38.8862 47.7369) (size 0.6) (drill 0.3) (layers "F.Cu" "B.Cu") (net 21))
 (segment (start 38.3318 71.9082) (end 37.22 73.02) (width 0.2) (layer "B.Cu") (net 21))
 (segment (start 38.3318 48.2913) (end 38.3318 71.9082) (width 0.2) (layer "B.Cu") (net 21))
 (segment (start 38.8862 47.7369) (end 38.3318 48.2913) (width 0.2) (layer "B.Cu") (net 21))
 (segment (start 38.8862 47.7369) (end 39.8977 48.7484) (width 0.2) (layer "B.Cu") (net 21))
 (segment (start 39.8977 48.7484) (end 38.8862 47.7369) (width 0.2) (layer "B.Cu") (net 21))
 (segment (start 37.22 62.86) (end 36.0712 64.0088) (width 0.2) (layer "F.Cu") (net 16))
 (segment (start 36.0712 64.0088) (end 36.0712 65.8183) (width 0.2) (layer "F.Cu") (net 16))
 (segment (start 36.0712 65.8183) (end 36.8169 66.564) (width 0.2) (layer "F.Cu") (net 16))
 (segment (start 66.877 66.564) (end 71.091 62.35) (width 0.2) (layer "F.Cu") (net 16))
 (segment (start 36.8169 66.564) (end 66.877 66.564) (width 0.2) (layer "F.Cu") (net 16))
 (segment (start 71.091 62.35) (end 87.92 62.35) (width 0.2) (layer "F.Cu") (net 16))
 (segment (start 65.1361 63.5661) (end 65.1361 75.2737) (width 0.2) (layer "B.Cu") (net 13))
 (segment (start 55 85.4098) (end 55 85.72) (width 0.2) (layer "B.Cu") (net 13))
 (segment (start 65.1361 75.2737) (end 55 85.4098) (width 0.2) (layer "B.Cu") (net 13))
 (segment (start 63.92 62.35) (end 65.1361 63.5661) (width 0.2) (layer "B.Cu") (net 13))
 (segment (start 55 80.64) (end 53.4923 79.1323) (width 0.2) (layer "B.Cu") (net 8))
 (segment (start 56.473 57.097) (end 63.92 49.65) (width 0.2) (layer "B.Cu") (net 8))
 (segment (start 53.4923 62.7824) (end 54.6847 61.59) (width 0.2) (layer "B.Cu") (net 8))
 (segment (start 54.6847 61.59) (end 55.2951 61.59) (width 0.2) (layer "B.Cu") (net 8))
 (segment (start 56.473 60.4121) (end 56.473 57.097) (width 0.2) (layer "B.Cu") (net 8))
 (segment (start 55.2951 61.59) (end 56.473 60.4121) (width 0.2) (layer "B.Cu") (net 8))
 (segment (start 53.4923 79.1323) (end 53.4923 62.7824) (width 0.2) (layer "B.Cu") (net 8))
 (segment (start 37.22 67.94) (end 38.3343 69.0543) (width 0.2) (layer "F.Cu") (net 17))
 (segment (start 89.0722 60.9622) (end 87.92 59.81) (width 0.2) (layer "F.Cu") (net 17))
 (segment (start 89.0722 62.8604) (end 89.0722 60.9622) (width 0.2) (layer "F.Cu") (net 17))
 (segment (start 88.3126 63.62) (end 89.0722 62.8604) (width 0.2) (layer "F.Cu") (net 17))
 (segment (start 77.6792 63.62) (end 88.3126 63.62) (width 0.2) (layer "F.Cu") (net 17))
 (segment (start 38.3343 69.0543) (end 72.2449 69.0543) (width 0.2) (layer "F.Cu") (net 17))
 (segment (start 72.2449 69.0543) (end 77.6792 63.62) (width 0.2) (layer "F.Cu") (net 17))
 (segment (start 65.5598 77.7002) (end 65.5598 48.7498) (width 0.2) (layer "B.Cu") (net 7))
 (segment (start 65.5598 48.7498) (end 63.92 47.11) (width 0.2) (layer "B.Cu") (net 7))
 (segment (start 55 88.26) (end 65.5598 77.7002) (width 0.2) (layer "B.Cu") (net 7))
 (segment (start 54.014365 60.89) (end 43.512 60.89) (width 0.2) (layer "F.Cu") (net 18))
 (segment (start 54.544365 61.42) (end 54.014365 60.89) (width 0.2) (layer "F.Cu") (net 18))
 (segment (start 59.4795 61.08) (end 59.1395 61.42) (width 0.2) (layer "F.Cu") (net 18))
 (segment (start 43.512 60.89) (end 41.2096 63.1924) (width 0.2) (layer "F.Cu") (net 18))
 (segment (start 84.11 61.08) (end 59.4795 61.08) (width 0.2) (layer "F.Cu") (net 18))
 (segment (start 59.1395 61.42) (end 54.544365 61.42) (width 0.2) (layer "F.Cu") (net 18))
 (segment (start 87.92 57.27) (end 84.11 61.08) (width 0.2) (layer "F.Cu") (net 18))
 (via (at 41.2096 63.1924) (size 0.6) (drill 0.3) (layers "F.Cu" "B.Cu") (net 18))
 (segment (start 38.6175 86.8625) (end 37.22 88.26) (width 0.2) (layer "B.Cu") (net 18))
 (segment (start 38.6175 80.253) (end 38.6175 86.8625) (width 0.2) (layer "B.Cu") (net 18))
 (segment (start 41.2096 63.1924) (end 41.2096 77.6609) (width 0.2) (layer "B.Cu") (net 18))
 (segment (start 41.2096 77.6609) (end 38.6175 80.253) (width 0.2) (layer "B.Cu") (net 18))
 (segment (start 66.1853 73.5315) (end 66.482 73.8282) (width 0.2) (layer "F.Cu") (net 22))
 (segment (start 64.5397 71.8859) (end 66.482 73.8282) (width 0.2) (layer "F.Cu") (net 22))
 (segment (start 40.8941 71.8859) (end 64.5397 71.8859) (width 0.2) (layer "F.Cu") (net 22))
 (segment (start 66.482 73.8282) (end 66.1853 73.5315) (width 0.2) (layer "F.Cu") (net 22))
 (segment (start 37.22 75.56) (end 40.8941 71.8859) (width 0.2) (layer "F.Cu") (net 22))
 (segment (start 87.2594 47.7706) (end 87.92 47.11) (width 0.2) (layer "F.Cu") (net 22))
 (segment (start 69.5209 47.7706) (end 87.2594 47.7706) (width 0.2) (layer "F.Cu") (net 22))
 (via (at 69.5209 47.7706) (size 0.6) (drill 0.3) (layers "F.Cu" "B.Cu") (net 22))
 (via (at 66.482 73.8282) (size 0.6) (drill 0.3) (layers "F.Cu" "B.Cu") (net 22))
 (segment (start 69.5209 47.7706) (end 66.482 50.8095) (width 0.2) (layer "B.Cu") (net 22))
 (segment (start 66.482 50.8095) (end 66.482 73.8282) (width 0.2) (layer "B.Cu") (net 22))
 (segment (start 66.1853 73.5315) (end 66.482 73.8282) (width 0.2) (layer "B.Cu") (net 22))
 (segment (start 66.482 73.8282) (end 66.1853 73.5315) (width 0.2) (layer "B.Cu") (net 22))
 (segment (start 63.92 59.81) (end 63.3073 59.1973) (width 0.2) (layer "F.Cu") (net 12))
 (segment (start 42.5026 59.1973) (end 37.22 64.4799) (width 0.2) (layer "F.Cu") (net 12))
 (segment (start 37.22 64.4799) (end 37.22 65.4) (width 0.2) (layer "F.Cu") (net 12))
 (segment (start 63.3073 59.1973) (end 42.5026 59.1973) (width 0.2) (layer "F.Cu") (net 12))
 (segment (start 38.6219 51.2981) (end 37.22 52.7) (width 0.2) (layer "F.Cu") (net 19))
 (segment (start 84.1948 51.0048) (end 59.3947 51.0048) (width 0.2) (layer "F.Cu") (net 19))
 (segment (start 87.92 54.73) (end 84.1948 51.0048) (width 0.2) (layer "F.Cu") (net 19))
 (segment (start 59.3947 51.0048) (end 59.1014 51.2981) (width 0.2) (layer "F.Cu") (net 19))
 (segment (start 59.1014 51.2981) (end 38.6219 51.2981) (width 0.2) (layer "F.Cu") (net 19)))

